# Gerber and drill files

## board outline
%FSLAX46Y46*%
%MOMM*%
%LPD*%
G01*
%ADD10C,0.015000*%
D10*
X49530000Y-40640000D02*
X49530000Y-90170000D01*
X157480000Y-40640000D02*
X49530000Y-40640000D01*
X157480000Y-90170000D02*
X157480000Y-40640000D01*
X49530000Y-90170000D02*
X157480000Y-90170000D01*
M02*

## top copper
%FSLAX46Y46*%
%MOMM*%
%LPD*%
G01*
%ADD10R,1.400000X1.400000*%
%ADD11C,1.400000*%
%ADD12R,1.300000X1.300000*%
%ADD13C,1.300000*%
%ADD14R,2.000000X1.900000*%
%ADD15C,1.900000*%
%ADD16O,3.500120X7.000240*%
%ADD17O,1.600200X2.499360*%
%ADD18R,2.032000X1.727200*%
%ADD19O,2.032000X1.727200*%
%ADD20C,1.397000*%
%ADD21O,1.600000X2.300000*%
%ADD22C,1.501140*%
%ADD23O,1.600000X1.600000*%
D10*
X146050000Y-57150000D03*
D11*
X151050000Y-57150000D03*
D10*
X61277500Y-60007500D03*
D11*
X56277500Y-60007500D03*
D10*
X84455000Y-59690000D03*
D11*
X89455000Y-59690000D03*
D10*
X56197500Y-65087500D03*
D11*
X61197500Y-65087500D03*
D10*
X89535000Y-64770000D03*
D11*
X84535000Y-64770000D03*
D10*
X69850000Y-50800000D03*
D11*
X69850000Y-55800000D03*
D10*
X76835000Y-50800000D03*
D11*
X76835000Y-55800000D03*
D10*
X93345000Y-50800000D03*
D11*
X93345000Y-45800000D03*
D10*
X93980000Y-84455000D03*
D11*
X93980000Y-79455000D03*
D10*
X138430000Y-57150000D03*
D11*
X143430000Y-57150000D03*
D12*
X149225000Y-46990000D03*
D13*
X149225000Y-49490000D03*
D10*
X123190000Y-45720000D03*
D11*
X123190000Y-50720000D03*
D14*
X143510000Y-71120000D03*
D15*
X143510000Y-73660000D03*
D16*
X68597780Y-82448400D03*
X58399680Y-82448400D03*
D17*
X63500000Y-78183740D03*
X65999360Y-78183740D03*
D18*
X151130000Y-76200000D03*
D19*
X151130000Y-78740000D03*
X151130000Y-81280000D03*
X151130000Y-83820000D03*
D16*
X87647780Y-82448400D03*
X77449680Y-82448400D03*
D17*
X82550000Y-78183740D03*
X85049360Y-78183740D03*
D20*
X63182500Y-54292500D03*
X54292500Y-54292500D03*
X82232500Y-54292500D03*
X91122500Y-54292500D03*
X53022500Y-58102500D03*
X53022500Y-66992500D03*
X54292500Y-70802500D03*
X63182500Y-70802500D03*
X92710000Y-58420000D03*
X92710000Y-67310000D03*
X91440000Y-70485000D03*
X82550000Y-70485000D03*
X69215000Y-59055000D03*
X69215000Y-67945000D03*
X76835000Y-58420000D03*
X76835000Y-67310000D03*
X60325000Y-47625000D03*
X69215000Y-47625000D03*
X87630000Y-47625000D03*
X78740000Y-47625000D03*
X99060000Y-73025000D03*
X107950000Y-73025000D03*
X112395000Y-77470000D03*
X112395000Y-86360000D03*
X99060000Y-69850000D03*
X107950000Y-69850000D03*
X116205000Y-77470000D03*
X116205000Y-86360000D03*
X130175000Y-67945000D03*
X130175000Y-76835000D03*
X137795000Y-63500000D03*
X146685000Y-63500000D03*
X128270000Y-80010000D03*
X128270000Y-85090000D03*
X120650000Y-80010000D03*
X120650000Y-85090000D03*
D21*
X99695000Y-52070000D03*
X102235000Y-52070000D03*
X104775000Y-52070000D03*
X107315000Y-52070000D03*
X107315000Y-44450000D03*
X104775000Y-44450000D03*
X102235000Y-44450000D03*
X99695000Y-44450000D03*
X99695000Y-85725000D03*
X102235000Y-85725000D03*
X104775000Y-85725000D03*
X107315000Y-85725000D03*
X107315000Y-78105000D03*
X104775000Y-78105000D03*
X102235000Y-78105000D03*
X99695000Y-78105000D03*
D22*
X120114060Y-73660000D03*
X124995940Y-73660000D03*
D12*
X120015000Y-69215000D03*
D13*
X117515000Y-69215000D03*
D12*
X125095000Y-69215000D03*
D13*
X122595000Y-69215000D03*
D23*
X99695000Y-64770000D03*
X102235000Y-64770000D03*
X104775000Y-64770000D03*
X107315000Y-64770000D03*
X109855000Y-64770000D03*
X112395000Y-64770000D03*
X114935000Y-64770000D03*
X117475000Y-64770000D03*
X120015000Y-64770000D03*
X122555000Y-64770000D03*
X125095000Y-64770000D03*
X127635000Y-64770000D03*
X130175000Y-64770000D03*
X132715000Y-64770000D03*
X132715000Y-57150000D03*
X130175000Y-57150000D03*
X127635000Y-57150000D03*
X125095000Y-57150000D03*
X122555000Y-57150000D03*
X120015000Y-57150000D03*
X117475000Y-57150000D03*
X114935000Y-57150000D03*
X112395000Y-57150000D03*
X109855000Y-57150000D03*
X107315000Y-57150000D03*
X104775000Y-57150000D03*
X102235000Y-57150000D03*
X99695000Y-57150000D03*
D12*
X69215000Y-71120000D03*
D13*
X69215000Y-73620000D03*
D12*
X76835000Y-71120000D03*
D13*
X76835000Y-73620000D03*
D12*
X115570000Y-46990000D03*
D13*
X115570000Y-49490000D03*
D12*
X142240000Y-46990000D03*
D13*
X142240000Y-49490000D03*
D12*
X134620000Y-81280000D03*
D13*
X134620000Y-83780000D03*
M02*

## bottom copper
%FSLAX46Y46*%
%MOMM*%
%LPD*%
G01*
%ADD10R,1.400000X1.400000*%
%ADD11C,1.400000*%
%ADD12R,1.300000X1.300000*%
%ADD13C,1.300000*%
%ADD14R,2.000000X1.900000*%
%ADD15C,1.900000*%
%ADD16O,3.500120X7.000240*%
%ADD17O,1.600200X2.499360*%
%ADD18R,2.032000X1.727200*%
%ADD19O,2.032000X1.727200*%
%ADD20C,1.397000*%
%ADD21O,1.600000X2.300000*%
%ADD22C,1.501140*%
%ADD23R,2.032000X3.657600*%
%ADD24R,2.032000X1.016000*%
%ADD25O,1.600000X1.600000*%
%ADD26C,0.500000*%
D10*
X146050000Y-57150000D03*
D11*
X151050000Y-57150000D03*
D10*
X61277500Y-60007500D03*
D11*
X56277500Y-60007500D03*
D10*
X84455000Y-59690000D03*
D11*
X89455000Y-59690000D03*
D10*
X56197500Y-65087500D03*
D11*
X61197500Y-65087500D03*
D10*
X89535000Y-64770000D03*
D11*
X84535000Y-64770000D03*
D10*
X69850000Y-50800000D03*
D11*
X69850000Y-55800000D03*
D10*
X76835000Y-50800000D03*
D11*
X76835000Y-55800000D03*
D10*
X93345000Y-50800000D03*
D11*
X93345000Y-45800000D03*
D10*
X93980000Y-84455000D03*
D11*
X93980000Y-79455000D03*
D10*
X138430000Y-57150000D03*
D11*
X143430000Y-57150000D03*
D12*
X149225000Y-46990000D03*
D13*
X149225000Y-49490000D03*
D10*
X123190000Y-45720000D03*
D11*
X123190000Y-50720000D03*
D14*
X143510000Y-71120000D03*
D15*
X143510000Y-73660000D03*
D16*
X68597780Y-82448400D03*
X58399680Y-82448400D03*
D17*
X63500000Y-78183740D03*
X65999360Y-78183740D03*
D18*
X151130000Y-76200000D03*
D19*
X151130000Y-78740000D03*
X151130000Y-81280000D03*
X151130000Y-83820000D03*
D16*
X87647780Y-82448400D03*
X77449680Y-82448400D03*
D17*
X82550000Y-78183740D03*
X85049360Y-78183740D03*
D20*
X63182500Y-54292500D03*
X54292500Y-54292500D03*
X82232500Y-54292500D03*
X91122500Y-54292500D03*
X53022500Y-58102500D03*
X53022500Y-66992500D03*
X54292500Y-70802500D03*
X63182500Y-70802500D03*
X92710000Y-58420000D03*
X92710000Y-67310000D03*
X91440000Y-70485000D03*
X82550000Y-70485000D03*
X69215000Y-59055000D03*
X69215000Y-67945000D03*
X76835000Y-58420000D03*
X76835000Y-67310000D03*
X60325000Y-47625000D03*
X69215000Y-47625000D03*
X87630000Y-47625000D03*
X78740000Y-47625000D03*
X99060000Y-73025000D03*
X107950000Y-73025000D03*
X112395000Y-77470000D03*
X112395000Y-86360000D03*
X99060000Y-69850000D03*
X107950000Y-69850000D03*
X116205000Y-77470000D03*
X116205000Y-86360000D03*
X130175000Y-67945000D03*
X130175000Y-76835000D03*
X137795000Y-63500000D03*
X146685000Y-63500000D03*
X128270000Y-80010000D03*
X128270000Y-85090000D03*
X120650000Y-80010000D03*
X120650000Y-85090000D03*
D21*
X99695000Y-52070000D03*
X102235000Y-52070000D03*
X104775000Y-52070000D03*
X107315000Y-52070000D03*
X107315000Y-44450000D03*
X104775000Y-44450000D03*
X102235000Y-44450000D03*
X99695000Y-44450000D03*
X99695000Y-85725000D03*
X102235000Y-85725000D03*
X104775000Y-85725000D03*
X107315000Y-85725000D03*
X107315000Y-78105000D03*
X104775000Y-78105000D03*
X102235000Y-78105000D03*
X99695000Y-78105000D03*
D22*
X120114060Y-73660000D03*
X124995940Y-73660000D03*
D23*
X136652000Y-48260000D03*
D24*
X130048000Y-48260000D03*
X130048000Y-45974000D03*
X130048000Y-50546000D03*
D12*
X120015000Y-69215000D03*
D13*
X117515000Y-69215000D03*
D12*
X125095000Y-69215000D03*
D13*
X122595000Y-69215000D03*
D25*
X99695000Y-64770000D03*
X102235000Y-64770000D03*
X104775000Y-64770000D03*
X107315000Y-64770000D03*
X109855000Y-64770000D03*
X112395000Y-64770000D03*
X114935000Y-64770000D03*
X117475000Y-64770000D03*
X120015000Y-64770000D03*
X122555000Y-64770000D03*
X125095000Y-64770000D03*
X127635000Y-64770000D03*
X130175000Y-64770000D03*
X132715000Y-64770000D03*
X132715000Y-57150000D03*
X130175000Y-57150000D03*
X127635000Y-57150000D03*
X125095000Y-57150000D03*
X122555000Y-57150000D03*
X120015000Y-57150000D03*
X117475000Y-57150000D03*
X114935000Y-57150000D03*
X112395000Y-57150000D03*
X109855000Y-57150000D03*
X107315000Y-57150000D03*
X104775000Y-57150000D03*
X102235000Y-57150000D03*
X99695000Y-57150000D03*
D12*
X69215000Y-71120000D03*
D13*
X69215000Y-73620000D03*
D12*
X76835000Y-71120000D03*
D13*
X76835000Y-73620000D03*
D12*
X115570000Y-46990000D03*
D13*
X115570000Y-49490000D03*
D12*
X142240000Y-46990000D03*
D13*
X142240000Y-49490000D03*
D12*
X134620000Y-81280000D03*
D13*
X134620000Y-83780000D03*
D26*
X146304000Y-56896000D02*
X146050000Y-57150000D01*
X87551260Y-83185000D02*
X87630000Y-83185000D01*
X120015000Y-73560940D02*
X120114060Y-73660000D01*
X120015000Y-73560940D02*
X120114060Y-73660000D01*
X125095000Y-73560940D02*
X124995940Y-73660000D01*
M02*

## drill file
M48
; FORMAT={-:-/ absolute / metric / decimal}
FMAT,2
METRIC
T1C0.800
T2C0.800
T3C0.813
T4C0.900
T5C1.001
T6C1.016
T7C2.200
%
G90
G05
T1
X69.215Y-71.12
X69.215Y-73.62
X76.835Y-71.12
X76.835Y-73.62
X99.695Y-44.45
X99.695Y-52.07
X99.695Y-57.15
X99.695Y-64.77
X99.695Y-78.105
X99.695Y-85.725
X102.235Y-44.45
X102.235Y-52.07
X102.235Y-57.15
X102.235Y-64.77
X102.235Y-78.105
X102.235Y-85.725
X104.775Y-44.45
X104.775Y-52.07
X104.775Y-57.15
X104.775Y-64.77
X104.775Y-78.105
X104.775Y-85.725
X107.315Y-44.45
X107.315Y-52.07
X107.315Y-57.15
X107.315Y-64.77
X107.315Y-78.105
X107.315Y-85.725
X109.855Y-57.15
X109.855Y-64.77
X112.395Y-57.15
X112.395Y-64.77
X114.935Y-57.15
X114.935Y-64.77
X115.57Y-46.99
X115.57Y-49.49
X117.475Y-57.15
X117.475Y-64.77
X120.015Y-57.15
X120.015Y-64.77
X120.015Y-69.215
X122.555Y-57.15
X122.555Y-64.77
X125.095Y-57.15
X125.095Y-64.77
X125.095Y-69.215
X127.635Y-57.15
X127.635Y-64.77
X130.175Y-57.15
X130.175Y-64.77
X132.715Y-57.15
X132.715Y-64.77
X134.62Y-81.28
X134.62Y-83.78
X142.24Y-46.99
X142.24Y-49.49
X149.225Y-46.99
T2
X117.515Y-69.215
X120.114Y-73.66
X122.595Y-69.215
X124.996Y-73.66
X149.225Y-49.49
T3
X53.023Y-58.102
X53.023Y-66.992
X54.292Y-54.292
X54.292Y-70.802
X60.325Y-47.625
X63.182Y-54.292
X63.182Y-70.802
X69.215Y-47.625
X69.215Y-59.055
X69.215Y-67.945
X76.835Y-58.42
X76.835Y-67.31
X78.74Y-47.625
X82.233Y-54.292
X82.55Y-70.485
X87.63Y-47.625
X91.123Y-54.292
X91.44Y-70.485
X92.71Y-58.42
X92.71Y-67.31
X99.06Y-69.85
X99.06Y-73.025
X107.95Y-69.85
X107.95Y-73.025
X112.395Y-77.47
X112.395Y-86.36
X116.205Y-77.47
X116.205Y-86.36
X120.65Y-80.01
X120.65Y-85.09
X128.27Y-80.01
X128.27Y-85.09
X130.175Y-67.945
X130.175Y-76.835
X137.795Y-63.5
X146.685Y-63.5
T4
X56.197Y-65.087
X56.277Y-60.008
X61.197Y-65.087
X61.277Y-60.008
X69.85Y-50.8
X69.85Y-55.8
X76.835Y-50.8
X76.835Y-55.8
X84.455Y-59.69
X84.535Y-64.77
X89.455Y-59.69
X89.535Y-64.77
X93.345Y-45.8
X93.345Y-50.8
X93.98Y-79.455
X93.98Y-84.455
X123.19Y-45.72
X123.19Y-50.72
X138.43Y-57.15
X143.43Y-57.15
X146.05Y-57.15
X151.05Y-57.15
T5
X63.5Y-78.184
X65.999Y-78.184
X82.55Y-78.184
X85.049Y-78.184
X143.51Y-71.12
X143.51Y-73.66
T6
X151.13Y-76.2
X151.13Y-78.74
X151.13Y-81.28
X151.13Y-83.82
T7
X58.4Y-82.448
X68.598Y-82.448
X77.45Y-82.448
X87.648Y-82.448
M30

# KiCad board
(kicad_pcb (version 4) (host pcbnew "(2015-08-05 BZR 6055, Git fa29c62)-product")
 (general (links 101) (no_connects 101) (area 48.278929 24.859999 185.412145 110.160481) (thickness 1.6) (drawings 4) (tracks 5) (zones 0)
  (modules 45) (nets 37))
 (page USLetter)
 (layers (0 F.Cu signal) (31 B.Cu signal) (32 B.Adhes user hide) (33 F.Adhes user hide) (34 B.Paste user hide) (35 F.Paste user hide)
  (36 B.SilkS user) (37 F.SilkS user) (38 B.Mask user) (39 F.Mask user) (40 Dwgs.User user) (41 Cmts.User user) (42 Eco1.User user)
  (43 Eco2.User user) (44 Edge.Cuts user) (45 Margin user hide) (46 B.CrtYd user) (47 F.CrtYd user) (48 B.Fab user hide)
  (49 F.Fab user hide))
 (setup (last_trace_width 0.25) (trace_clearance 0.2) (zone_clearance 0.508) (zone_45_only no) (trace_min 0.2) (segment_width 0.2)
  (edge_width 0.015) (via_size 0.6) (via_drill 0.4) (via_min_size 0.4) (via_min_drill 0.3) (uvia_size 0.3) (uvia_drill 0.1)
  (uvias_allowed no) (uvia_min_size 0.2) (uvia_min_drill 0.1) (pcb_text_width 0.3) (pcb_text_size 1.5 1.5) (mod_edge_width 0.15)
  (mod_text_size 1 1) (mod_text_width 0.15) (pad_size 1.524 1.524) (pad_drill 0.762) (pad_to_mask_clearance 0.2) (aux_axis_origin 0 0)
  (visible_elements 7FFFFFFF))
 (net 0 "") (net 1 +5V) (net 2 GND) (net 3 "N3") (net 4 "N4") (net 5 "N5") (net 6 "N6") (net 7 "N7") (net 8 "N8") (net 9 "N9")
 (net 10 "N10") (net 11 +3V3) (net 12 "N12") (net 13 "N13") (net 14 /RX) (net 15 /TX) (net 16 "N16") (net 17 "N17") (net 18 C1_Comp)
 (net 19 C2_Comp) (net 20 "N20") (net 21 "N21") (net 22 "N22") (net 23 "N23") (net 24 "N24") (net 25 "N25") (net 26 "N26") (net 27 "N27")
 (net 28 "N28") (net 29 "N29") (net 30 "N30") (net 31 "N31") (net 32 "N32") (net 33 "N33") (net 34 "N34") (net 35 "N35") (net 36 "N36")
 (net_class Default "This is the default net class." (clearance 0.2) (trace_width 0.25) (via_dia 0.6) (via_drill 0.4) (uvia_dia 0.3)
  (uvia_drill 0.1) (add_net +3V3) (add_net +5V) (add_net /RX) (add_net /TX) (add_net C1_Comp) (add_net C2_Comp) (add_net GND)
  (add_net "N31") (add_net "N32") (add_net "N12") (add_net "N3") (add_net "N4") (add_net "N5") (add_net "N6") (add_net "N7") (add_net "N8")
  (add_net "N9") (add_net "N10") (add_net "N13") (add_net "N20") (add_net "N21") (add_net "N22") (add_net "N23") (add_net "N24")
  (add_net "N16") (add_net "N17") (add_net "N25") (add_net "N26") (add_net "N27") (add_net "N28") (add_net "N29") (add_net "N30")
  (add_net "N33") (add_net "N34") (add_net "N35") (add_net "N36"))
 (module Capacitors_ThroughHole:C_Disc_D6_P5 (layer F.Cu) (at 146.05 57.15)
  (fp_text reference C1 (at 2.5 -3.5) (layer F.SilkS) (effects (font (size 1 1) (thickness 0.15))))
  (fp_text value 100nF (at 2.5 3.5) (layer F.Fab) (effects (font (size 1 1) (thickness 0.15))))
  (pad 1 thru_hole rect (at 0 0) (size 1.4 1.4) (drill 0.9) (layers *.Cu *.Mask F.SilkS) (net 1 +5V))
  (pad 2 thru_hole circle (at 5 0) (size 1.4 1.4) (drill 0.9) (layers *.Cu *.Mask F.SilkS) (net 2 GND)))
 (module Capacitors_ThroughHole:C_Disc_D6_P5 (layer F.Cu) (at 61.2775 60.0075 180)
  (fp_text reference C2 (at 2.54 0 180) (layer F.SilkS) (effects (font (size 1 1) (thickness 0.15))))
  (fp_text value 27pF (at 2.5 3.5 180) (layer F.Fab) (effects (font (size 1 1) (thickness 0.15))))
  (pad 1 thru_hole rect (at 0 0 180) (size 1.4 1.4) (drill 0.9) (layers *.Cu *.Mask F.SilkS) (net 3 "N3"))
  (pad 2 thru_hole circle (at 5 0 180) (size 1.4 1.4) (drill 0.9) (layers *.Cu *.Mask F.SilkS) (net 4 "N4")))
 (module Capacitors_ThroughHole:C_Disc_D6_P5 (layer F.Cu) (at 84.455 59.69)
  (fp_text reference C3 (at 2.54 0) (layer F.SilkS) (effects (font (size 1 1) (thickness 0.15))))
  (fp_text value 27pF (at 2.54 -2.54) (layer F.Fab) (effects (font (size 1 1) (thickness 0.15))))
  (pad 1 thru_hole rect (at 0 0) (size 1.4 1.4) (drill 0.9) (layers *.Cu *.Mask F.SilkS) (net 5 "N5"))
  (pad 2 thru_hole circle (at 5 0) (size 1.4 1.4) (drill 0.9) (layers *.Cu *.Mask F.SilkS) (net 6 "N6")))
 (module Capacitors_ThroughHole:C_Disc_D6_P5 (layer F.Cu) (at 56.1975 65.0875)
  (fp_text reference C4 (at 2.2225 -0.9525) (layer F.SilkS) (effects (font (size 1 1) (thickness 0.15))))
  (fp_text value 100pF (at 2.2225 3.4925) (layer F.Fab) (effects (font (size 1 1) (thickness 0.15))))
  (pad 1 thru_hole rect (at 0 0) (size 1.4 1.4) (drill 0.9) (layers *.Cu *.Mask F.SilkS) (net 4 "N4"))
  (pad 2 thru_hole circle (at 5 0) (size 1.4 1.4) (drill 0.9) (layers *.Cu *.Mask F.SilkS) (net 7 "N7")))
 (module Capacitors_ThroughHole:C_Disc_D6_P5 (layer F.Cu) (at 89.535 64.77 180)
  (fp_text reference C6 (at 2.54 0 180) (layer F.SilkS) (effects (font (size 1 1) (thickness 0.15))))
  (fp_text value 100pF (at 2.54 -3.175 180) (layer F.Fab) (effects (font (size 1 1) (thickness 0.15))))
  (pad 1 thru_hole rect (at 0 0 180) (size 1.4 1.4) (drill 0.9) (layers *.Cu *.Mask F.SilkS) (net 6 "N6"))
  (pad 2 thru_hole circle (at 5 0 180) (size 1.4 1.4) (drill 0.9) (layers *.Cu *.Mask F.SilkS) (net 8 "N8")))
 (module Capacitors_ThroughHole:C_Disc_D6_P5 (layer F.Cu) (at 69.85 50.8 270)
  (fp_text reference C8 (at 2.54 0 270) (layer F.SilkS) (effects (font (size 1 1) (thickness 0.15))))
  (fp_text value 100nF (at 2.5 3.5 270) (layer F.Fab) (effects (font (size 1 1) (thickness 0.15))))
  (pad 1 thru_hole rect (at 0 0 270) (size 1.4 1.4) (drill 0.9) (layers *.Cu *.Mask F.SilkS) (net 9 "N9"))
  (pad 2 thru_hole circle (at 5 0 270) (size 1.4 1.4) (drill 0.9) (layers *.Cu *.Mask F.SilkS) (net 2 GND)))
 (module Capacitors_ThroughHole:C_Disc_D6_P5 (layer F.Cu) (at 76.835 50.8 270)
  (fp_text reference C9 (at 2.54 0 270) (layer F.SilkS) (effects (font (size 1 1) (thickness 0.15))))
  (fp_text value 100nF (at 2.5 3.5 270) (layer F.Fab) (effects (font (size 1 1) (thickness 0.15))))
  (pad 1 thru_hole rect (at 0 0 270) (size 1.4 1.4) (drill 0.9) (layers *.Cu *.Mask F.SilkS) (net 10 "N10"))
  (pad 2 thru_hole circle (at 5 0 270) (size 1.4 1.4) (drill 0.9) (layers *.Cu *.Mask F.SilkS) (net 2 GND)))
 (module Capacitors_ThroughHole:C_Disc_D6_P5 (layer F.Cu) (at 93.345 50.8 90)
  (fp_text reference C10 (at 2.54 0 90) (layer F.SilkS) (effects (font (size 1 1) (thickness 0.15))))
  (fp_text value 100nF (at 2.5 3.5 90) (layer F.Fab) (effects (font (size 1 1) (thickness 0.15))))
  (pad 1 thru_hole rect (at 0 0 90) (size 1.4 1.4) (drill 0.9) (layers *.Cu *.Mask F.SilkS) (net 2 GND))
  (pad 2 thru_hole circle (at 5 0 90) (size 1.4 1.4) (drill 0.9) (layers *.Cu *.Mask F.SilkS) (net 1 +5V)))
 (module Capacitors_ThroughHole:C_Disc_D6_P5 (layer F.Cu) (at 93.98 84.455 90)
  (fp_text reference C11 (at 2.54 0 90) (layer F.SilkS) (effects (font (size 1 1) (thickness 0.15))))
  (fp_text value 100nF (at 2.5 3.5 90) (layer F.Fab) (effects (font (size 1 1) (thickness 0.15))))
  (pad 1 thru_hole rect (at 0 0 90) (size 1.4 1.4) (drill 0.9) (layers *.Cu *.Mask F.SilkS) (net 2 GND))
  (pad 2 thru_hole circle (at 5 0 90) (size 1.4 1.4) (drill 0.9) (layers *.Cu *.Mask F.SilkS) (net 1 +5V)))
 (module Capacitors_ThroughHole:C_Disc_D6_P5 (layer F.Cu) (at 138.43 57.15)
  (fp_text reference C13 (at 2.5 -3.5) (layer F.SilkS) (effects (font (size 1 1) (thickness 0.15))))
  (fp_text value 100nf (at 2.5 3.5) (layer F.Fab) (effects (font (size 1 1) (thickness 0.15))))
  (pad 1 thru_hole rect (at 0 0) (size 1.4 1.4) (drill 0.9) (layers *.Cu *.Mask F.SilkS) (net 1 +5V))
  (pad 2 thru_hole circle (at 5 0) (size 1.4 1.4) (drill 0.9) (layers *.Cu *.Mask F.SilkS) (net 2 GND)))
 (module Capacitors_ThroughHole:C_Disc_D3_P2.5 (layer F.Cu) (at 149.225 46.99 270)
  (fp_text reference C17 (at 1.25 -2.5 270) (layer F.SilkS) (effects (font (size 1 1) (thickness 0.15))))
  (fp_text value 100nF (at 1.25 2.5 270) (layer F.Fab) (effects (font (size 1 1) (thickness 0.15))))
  (pad 1 thru_hole rect (at 0 0 270) (size 1.3 1.3) (drill 0.8) (layers *.Cu *.Mask F.SilkS) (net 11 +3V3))
  (pad 2 thru_hole circle (at 2.5 0 270) (size 1.3 1.3) (drill 0.8001) (layers *.Cu *.Mask F.SilkS) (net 2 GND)))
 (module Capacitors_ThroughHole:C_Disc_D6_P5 (layer F.Cu) (at 123.19 45.72 270)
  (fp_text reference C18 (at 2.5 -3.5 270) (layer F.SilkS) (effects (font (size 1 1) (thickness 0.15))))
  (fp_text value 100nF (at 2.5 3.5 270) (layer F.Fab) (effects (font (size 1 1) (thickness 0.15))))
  (pad 1 thru_hole rect (at 0 0 270) (size 1.4 1.4) (drill 0.9) (layers *.Cu *.Mask F.SilkS) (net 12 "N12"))
  (pad 2 thru_hole circle (at 5 0 270) (size 1.4 1.4) (drill 0.9) (layers *.Cu *.Mask F.SilkS) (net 2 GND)))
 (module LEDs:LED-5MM (layer F.Cu) (at 143.51 71.12 270)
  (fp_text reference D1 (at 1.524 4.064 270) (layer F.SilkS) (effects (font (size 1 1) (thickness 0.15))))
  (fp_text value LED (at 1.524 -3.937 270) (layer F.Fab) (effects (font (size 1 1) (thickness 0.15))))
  (pad 1 thru_hole rect (at 0 0) (size 2 1.9) (drill 1.00076) (layers *.Cu *.Mask F.SilkS) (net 2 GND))
  (pad 2 thru_hole circle (at 2.54 0 270) (size 1.9 1.9) (drill 1.00076) (layers *.Cu *.Mask F.SilkS) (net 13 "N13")))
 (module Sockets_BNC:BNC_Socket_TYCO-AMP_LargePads (layer F.Cu) (at 63.5 83.185 180)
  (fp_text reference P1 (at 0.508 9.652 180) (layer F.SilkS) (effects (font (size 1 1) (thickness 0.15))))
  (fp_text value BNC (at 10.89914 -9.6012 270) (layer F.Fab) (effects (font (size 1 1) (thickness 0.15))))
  (pad 2 thru_hole oval (at -5.09778 0.7366 180) (size 3.50012 7.00024) (drill 2.19964) (layers *.Cu *.Mask F.SilkS) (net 2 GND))
  (pad 2 thru_hole oval (at 5.10032 0.7366 180) (size 3.50012 7.00024) (drill 2.19964) (layers *.Cu *.Mask F.SilkS) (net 2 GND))
  (pad 1 thru_hole oval (at 0 5.00126 180) (size 1.6002 2.49936) (drill 1.00076) (layers *.Cu *.Mask F.SilkS) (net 3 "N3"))
  (pad 2 thru_hole oval (at -2.49936 5.00126 180) (size 1.6002 2.49936) (drill 1.00076) (layers *.Cu *.Mask F.SilkS) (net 2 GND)))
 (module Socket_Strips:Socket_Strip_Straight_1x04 (layer F.Cu) (at 151.13 76.2 270)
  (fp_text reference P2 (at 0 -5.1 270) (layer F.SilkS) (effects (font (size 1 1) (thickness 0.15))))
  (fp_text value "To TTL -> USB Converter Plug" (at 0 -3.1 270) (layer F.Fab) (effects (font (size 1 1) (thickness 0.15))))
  (pad 1 thru_hole rect (at 0 0 270) (size 1.7272 2.032) (drill 1.016) (layers *.Cu *.Mask F.SilkS) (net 2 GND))
  (pad 2 thru_hole oval (at 2.54 0 270) (size 1.7272 2.032) (drill 1.016) (layers *.Cu *.Mask F.SilkS) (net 1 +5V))
  (pad 3 thru_hole oval (at 5.08 0 270) (size 1.7272 2.032) (drill 1.016) (layers *.Cu *.Mask F.SilkS) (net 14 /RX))
  (pad 4 thru_hole oval (at 7.62 0 270) (size 1.7272 2.032) (drill 1.016) (layers *.Cu *.Mask F.SilkS) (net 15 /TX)))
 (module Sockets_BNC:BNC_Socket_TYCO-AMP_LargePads (layer F.Cu) (at 82.55 83.185 180)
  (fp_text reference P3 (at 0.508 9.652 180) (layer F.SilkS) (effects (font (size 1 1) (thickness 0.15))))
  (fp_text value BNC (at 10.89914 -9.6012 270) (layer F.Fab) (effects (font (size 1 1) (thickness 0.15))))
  (pad 2 thru_hole oval (at -5.09778 0.7366 180) (size 3.50012 7.00024) (drill 2.19964) (layers *.Cu *.Mask F.SilkS) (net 2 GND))
  (pad 2 thru_hole oval (at 5.10032 0.7366 180) (size 3.50012 7.00024) (drill 2.19964) (layers *.Cu *.Mask F.SilkS) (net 2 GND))
  (pad 1 thru_hole oval (at 0 5.00126 180) (size 1.6002 2.49936) (drill 1.00076) (layers *.Cu *.Mask F.SilkS) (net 5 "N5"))
  (pad 2 thru_hole oval (at -2.49936 5.00126 180) (size 1.6002 2.49936) (drill 1.00076) (layers *.Cu *.Mask F.SilkS) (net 2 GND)))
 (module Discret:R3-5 (layer F.Cu) (at 58.7375 54.2925 180)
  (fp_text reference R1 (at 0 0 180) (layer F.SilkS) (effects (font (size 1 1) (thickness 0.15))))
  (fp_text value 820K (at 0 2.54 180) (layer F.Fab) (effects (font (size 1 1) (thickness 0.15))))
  (pad 1 thru_hole circle (at -4.445 0 180) (size 1.397 1.397) (drill 0.8128) (layers *.Cu *.Mask F.SilkS) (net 3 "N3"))
  (pad 2 thru_hole circle (at 4.445 0 180) (size 1.397 1.397) (drill 0.8128) (layers *.Cu *.Mask F.SilkS) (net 4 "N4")))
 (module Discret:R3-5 (layer F.Cu) (at 86.6775 54.2925)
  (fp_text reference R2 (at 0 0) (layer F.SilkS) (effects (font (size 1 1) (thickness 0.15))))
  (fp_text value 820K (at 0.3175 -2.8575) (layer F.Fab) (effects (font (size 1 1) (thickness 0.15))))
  (pad 1 thru_hole circle (at -4.445 0) (size 1.397 1.397) (drill 0.8128) (layers *.Cu *.Mask F.SilkS) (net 5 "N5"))
  (pad 2 thru_hole circle (at 4.445 0) (size 1.397 1.397) (drill 0.8128) (layers *.Cu *.Mask F.SilkS) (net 6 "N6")))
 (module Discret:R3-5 (layer F.Cu) (at 53.0225 62.5475 270)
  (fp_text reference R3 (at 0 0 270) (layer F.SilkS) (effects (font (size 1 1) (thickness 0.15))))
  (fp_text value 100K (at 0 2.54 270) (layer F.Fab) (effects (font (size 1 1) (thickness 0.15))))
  (pad 1 thru_hole circle (at -4.445 0 270) (size 1.397 1.397) (drill 0.8128) (layers *.Cu *.Mask F.SilkS) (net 4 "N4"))
  (pad 2 thru_hole circle (at 4.445 0 270) (size 1.397 1.397) (drill 0.8128) (layers *.Cu *.Mask F.SilkS) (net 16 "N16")))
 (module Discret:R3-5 (layer F.Cu) (at 58.7375 70.8025)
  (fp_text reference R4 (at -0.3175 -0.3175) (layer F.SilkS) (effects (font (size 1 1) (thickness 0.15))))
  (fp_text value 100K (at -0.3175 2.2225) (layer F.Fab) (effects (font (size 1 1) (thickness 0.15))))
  (pad 1 thru_hole circle (at -4.445 0) (size 1.397 1.397) (drill 0.8128) (layers *.Cu *.Mask F.SilkS) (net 16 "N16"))
  (pad 2 thru_hole circle (at 4.445 0) (size 1.397 1.397) (drill 0.8128) (layers *.Cu *.Mask F.SilkS) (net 7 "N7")))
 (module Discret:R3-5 (layer F.Cu) (at 92.71 62.865 270)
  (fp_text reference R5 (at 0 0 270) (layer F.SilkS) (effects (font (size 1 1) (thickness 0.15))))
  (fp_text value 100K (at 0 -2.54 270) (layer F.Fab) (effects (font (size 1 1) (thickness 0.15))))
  (pad 1 thru_hole circle (at -4.445 0 270) (size 1.397 1.397) (drill 0.8128) (layers *.Cu *.Mask F.SilkS) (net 6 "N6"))
  (pad 2 thru_hole circle (at 4.445 0 270) (size 1.397 1.397) (drill 0.8128) (layers *.Cu *.Mask F.SilkS) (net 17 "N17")))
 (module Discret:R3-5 (layer F.Cu) (at 86.995 70.485 180)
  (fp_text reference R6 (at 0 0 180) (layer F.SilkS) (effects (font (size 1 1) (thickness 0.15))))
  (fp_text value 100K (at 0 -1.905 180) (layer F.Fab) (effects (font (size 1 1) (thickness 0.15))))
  (pad 1 thru_hole circle (at -4.445 0 180) (size 1.397 1.397) (drill 0.8128) (layers *.Cu *.Mask F.SilkS) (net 17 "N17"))
  (pad 2 thru_hole circle (at 4.445 0 180) (size 1.397 1.397) (drill 0.8128) (layers *.Cu *.Mask F.SilkS) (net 8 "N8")))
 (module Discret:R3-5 (layer F.Cu) (at 69.215 63.5 270)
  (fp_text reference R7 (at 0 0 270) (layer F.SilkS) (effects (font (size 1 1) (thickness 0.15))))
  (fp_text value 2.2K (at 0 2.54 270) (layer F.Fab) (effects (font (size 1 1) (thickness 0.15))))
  (pad 1 thru_hole circle (at -4.445 0 270) (size 1.397 1.397) (drill 0.8128) (layers *.Cu *.Mask F.SilkS) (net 9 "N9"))
  (pad 2 thru_hole circle (at 4.445 0 270) (size 1.397 1.397) (drill 0.8128) (layers *.Cu *.Mask F.SilkS) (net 7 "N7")))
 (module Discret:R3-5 (layer F.Cu) (at 76.835 62.865 270)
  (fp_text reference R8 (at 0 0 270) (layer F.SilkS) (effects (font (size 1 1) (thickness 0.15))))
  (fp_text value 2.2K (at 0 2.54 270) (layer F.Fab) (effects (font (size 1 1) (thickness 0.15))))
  (pad 1 thru_hole circle (at -4.445 0 270) (size 1.397 1.397) (drill 0.8128) (layers *.Cu *.Mask F.SilkS) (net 10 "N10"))
  (pad 2 thru_hole circle (at 4.445 0 270) (size 1.397 1.397) (drill 0.8128) (layers *.Cu *.Mask F.SilkS) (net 8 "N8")))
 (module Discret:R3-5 (layer F.Cu) (at 64.77 47.625)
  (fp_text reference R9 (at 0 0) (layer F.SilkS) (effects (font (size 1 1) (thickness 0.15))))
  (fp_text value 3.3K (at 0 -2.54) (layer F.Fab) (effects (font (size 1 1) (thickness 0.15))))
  (pad 1 thru_hole circle (at -4.445 0) (size 1.397 1.397) (drill 0.8128) (layers *.Cu *.Mask F.SilkS) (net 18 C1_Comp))
  (pad 2 thru_hole circle (at 4.445 0) (size 1.397 1.397) (drill 0.8128) (layers *.Cu *.Mask F.SilkS) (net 9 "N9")))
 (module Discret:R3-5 (layer F.Cu) (at 83.185 47.625 180)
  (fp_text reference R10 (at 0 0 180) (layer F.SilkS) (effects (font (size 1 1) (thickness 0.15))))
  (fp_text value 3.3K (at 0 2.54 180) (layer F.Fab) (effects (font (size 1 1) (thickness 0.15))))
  (pad 1 thru_hole circle (at -4.445 0 180) (size 1.397 1.397) (drill 0.8128) (layers *.Cu *.Mask F.SilkS) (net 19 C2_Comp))
  (pad 2 thru_hole circle (at 4.445 0 180) (size 1.397 1.397) (drill 0.8128) (layers *.Cu *.Mask F.SilkS) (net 10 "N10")))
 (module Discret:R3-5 (layer F.Cu) (at 103.505 73.025)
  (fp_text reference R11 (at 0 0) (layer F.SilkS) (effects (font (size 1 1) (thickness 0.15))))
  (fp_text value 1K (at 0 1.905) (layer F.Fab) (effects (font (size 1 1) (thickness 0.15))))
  (pad 1 thru_hole circle (at -4.445 0) (size 1.397 1.397) (drill 0.8128) (layers *.Cu *.Mask F.SilkS) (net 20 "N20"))
  (pad 2 thru_hole circle (at 4.445 0) (size 1.397 1.397) (drill 0.8128) (layers *.Cu *.Mask F.SilkS) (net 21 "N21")))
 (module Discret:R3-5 (layer F.Cu) (at 112.395 81.915 270)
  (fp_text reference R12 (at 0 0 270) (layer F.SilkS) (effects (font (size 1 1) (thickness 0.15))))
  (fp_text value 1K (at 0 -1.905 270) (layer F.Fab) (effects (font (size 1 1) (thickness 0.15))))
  (pad 1 thru_hole circle (at -4.445 0 270) (size 1.397 1.397) (drill 0.8128) (layers *.Cu *.Mask F.SilkS) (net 21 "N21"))
  (pad 2 thru_hole circle (at 4.445 0 270) (size 1.397 1.397) (drill 0.8128) (layers *.Cu *.Mask F.SilkS) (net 2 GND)))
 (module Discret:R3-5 (layer F.Cu) (at 103.505 69.85)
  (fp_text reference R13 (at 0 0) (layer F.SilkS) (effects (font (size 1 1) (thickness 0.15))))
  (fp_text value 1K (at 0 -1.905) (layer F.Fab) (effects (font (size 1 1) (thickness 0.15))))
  (pad 1 thru_hole circle (at -4.445 0) (size 1.397 1.397) (drill 0.8128) (layers *.Cu *.Mask F.SilkS) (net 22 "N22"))
  (pad 2 thru_hole circle (at 4.445 0) (size 1.397 1.397) (drill 0.8128) (layers *.Cu *.Mask F.SilkS) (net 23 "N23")))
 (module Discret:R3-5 (layer F.Cu) (at 116.205 81.915 270)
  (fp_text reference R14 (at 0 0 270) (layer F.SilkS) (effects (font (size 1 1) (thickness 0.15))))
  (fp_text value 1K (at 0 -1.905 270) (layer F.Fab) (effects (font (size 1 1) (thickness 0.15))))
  (pad 1 thru_hole circle (at -4.445 0 270) (size 1.397 1.397) (drill 0.8128) (layers *.Cu *.Mask F.SilkS) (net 23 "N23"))
  (pad 2 thru_hole circle (at 4.445 0 270) (size 1.397 1.397) (drill 0.8128) (layers *.Cu *.Mask F.SilkS) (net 2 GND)))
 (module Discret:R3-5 (layer F.Cu) (at 130.175 72.39 270)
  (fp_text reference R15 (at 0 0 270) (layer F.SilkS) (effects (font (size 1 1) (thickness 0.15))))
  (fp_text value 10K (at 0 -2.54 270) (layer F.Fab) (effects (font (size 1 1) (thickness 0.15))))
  (pad 1 thru_hole circle (at -4.445 0 270) (size 1.397 1.397) (drill 0.8128) (layers *.Cu *.Mask F.SilkS) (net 1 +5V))
  (pad 2 thru_hole circle (at 4.445 0 270) (size 1.397 1.397) (drill 0.8128) (layers *.Cu *.Mask F.SilkS) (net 12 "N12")))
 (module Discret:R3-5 (layer F.Cu) (at 142.24 63.5)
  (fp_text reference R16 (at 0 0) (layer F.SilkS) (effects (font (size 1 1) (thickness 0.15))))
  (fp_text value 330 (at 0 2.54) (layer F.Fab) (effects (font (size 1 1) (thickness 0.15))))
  (pad 1 thru_hole circle (at -4.445 0) (size 1.397 1.397) (drill 0.8128) (layers *.Cu *.Mask F.SilkS) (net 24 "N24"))
  (pad 2 thru_hole circle (at 4.445 0) (size 1.397 1.397) (drill 0.8128) (layers *.Cu *.Mask F.SilkS) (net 13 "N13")))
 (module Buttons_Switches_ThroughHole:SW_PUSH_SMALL (layer F.Cu) (at 124.46 82.55)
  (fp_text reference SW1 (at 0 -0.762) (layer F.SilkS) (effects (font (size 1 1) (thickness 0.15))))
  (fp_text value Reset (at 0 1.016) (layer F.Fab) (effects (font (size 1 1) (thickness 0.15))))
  (pad 1 thru_hole circle (at 3.81 -2.54) (size 1.397 1.397) (drill 0.8128) (layers *.Cu *.Mask F.SilkS) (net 12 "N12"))
  (pad 2 thru_hole circle (at 3.81 2.54) (size 1.397 1.397) (drill 0.8128) (layers *.Cu *.Mask F.SilkS) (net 2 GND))
  (pad 1 thru_hole circle (at -3.81 -2.54) (size 1.397 1.397) (drill 0.8128) (layers *.Cu *.Mask F.SilkS) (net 12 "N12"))
  (pad 2 thru_hole circle (at -3.81 2.54) (size 1.397 1.397) (drill 0.8128) (layers *.Cu *.Mask F.SilkS) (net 2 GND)))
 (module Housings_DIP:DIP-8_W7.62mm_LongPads (layer F.Cu) (at 99.695 52.07 90)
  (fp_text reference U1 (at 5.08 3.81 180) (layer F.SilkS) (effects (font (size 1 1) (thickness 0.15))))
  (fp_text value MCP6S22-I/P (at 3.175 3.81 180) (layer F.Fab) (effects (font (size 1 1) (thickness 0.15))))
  (pad 1 thru_hole oval (at 0 0 90) (size 2.3 1.6) (drill 0.8) (layers *.Cu *.Mask F.SilkS) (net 20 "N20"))
  (pad 2 thru_hole oval (at 0 2.54 90) (size 2.3 1.6) (drill 0.8) (layers *.Cu *.Mask F.SilkS) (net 4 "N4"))
  (pad 3 thru_hole oval (at 0 5.08 90) (size 2.3 1.6) (drill 0.8) (layers *.Cu *.Mask F.SilkS) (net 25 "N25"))
  (pad 4 thru_hole oval (at 0 7.62 90) (size 2.3 1.6) (drill 0.8) (layers *.Cu *.Mask F.SilkS) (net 2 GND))
  (pad 5 thru_hole oval (at 7.62 7.62 90) (size 2.3 1.6) (drill 0.8) (layers *.Cu *.Mask F.SilkS) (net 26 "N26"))
  (pad 6 thru_hole oval (at 7.62 5.08 90) (size 2.3 1.6) (drill 0.8) (layers *.Cu *.Mask F.SilkS) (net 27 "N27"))
  (pad 7 thru_hole oval (at 7.62 2.54 90) (size 2.3 1.6) (drill 0.8) (layers *.Cu *.Mask F.SilkS) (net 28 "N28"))
  (pad 8 thru_hole oval (at 7.62 0 90) (size 2.3 1.6) (drill 0.8) (layers *.Cu *.Mask F.SilkS) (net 1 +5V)))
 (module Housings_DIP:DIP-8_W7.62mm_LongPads (layer F.Cu) (at 99.695 85.725 90)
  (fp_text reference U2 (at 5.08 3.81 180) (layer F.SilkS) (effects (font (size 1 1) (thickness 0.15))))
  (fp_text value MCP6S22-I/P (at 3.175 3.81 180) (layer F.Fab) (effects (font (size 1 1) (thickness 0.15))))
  (pad 1 thru_hole oval (at 0 0 90) (size 2.3 1.6) (drill 0.8) (layers *.Cu *.Mask F.SilkS) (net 22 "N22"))
  (pad 2 thru_hole oval (at 0 2.54 90) (size 2.3 1.6) (drill 0.8) (layers *.Cu *.Mask F.SilkS) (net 6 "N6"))
  (pad 3 thru_hole oval (at 0 5.08 90) (size 2.3 1.6) (drill 0.8) (layers *.Cu *.Mask F.SilkS) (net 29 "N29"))
  (pad 4 thru_hole oval (at 0 7.62 90) (size 2.3 1.6) (drill 0.8) (layers *.Cu *.Mask F.SilkS) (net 2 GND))
  (pad 5 thru_hole oval (at 7.62 7.62 90) (size 2.3 1.6) (drill 0.8) (layers *.Cu *.Mask F.SilkS) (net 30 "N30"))
  (pad 6 thru_hole oval (at 7.62 5.08 90) (size 2.3 1.6) (drill 0.8) (layers *.Cu *.Mask F.SilkS) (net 27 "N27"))
  (pad 7 thru_hole oval (at 7.62 2.54 90) (size 2.3 1.6) (drill 0.8) (layers *.Cu *.Mask F.SilkS) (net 28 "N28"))
  (pad 8 thru_hole oval (at 7.62 0 90) (size 2.3 1.6) (drill 0.8) (layers *.Cu *.Mask F.SilkS) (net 1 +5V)))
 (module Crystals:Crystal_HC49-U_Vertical (layer F.Cu) (at 122.555 73.66)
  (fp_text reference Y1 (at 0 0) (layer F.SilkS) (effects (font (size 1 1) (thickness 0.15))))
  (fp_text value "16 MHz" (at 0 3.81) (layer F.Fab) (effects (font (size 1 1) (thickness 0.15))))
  (pad 1 thru_hole circle (at -2.44094 0) (size 1.50114 1.50114) (drill 0.8001) (layers *.Cu *.Mask F.SilkS) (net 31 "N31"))
  (pad 2 thru_hole circle (at 2.44094 0) (size 1.50114 1.50114) (drill 0.8001) (layers *.Cu *.Mask F.SilkS) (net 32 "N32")))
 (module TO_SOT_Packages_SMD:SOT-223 (layer B.Cu) (at 133.35 48.26 90)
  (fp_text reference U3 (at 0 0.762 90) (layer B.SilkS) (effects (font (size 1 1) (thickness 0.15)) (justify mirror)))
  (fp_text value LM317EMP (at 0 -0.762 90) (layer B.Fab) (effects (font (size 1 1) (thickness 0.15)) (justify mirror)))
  (pad 4 smd rect (at 0 3.302 90) (size 3.6576 2.032) (layers B.Cu B.Paste B.Mask))
  (pad 2 smd rect (at 0 -3.302 90) (size 1.016 2.032) (layers B.Cu B.Paste B.Mask) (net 11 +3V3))
  (pad 3 smd rect (at 2.286 -3.302 90) (size 1.016 2.032) (layers B.Cu B.Paste B.Mask) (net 1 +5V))
  (pad 1 smd rect (at -2.286 -3.302 90) (size 1.016 2.032) (layers B.Cu B.Paste B.Mask) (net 2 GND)))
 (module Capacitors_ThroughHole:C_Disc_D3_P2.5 (layer F.Cu) (at 120.015 69.215 180)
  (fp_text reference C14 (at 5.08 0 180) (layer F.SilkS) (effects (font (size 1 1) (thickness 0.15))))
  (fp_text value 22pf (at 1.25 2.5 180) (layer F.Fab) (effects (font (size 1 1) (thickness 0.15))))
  (pad 1 thru_hole rect (at 0 0 180) (size 1.3 1.3) (drill 0.8) (layers *.Cu *.Mask F.SilkS) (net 31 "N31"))
  (pad 2 thru_hole circle (at 2.5 0 180) (size 1.3 1.3) (drill 0.8001) (layers *.Cu *.Mask F.SilkS) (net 2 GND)))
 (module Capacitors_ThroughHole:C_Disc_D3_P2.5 (layer F.Cu) (at 125.095 69.215 180)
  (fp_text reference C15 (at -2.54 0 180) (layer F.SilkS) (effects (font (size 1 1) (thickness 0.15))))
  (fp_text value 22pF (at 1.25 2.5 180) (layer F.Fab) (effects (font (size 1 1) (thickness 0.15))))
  (pad 1 thru_hole rect (at 0 0 180) (size 1.3 1.3) (drill 0.8) (layers *.Cu *.Mask F.SilkS) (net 32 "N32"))
  (pad 2 thru_hole circle (at 2.5 0 180) (size 1.3 1.3) (drill 0.8001) (layers *.Cu *.Mask F.SilkS) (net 2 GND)))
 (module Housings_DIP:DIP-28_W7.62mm (layer F.Cu) (at 99.695 64.77 90)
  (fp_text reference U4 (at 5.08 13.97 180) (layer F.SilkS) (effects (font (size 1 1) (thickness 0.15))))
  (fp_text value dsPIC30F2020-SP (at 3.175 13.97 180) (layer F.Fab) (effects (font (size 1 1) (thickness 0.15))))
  (pad 1 thru_hole oval (at 0 0 90) (size 1.6 1.6) (drill 0.8) (layers *.Cu *.Mask F.SilkS) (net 12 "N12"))
  (pad 2 thru_hole oval (at 0 2.54 90) (size 1.6 1.6) (drill 0.8) (layers *.Cu *.Mask F.SilkS) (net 20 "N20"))
  (pad 3 thru_hole oval (at 0 5.08 90) (size 1.6 1.6) (drill 0.8) (layers *.Cu *.Mask F.SilkS) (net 22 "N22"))
  (pad 4 thru_hole oval (at 0 7.62 90) (size 1.6 1.6) (drill 0.8) (layers *.Cu *.Mask F.SilkS) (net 11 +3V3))
  (pad 5 thru_hole oval (at 0 10.16 90) (size 1.6 1.6) (drill 0.8) (layers *.Cu *.Mask F.SilkS) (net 11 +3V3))
  (pad 6 thru_hole oval (at 0 12.7 90) (size 1.6 1.6) (drill 0.8) (layers *.Cu *.Mask F.SilkS) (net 21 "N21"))
  (pad 7 thru_hole oval (at 0 15.24 90) (size 1.6 1.6) (drill 0.8) (layers *.Cu *.Mask F.SilkS) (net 23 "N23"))
  (pad 8 thru_hole oval (at 0 17.78 90) (size 1.6 1.6) (drill 0.8) (layers *.Cu *.Mask F.SilkS) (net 2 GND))
  (pad 9 thru_hole oval (at 0 20.32 90) (size 1.6 1.6) (drill 0.8) (layers *.Cu *.Mask F.SilkS) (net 31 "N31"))
  (pad 10 thru_hole oval (at 0 22.86 90) (size 1.6 1.6) (drill 0.8) (layers *.Cu *.Mask F.SilkS) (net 32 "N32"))
  (pad 11 thru_hole oval (at 0 25.4 90) (size 1.6 1.6) (drill 0.8) (layers *.Cu *.Mask F.SilkS) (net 15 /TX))
  (pad 12 thru_hole oval (at 0 27.94 90) (size 1.6 1.6) (drill 0.8) (layers *.Cu *.Mask F.SilkS) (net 14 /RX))
  (pad 13 thru_hole oval (at 0 30.48 90) (size 1.6 1.6) (drill 0.8) (layers *.Cu *.Mask F.SilkS) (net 1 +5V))
  (pad 14 thru_hole oval (at 0 33.02 90) (size 1.6 1.6) (drill 0.8) (layers *.Cu *.Mask F.SilkS) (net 19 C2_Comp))
  (pad 15 thru_hole oval (at 7.62 33.02 90) (size 1.6 1.6) (drill 0.8) (layers *.Cu *.Mask F.SilkS) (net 18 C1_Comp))
  (pad 16 thru_hole oval (at 7.62 30.48 90) (size 1.6 1.6) (drill 0.8) (layers *.Cu *.Mask F.SilkS) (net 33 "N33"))
  (pad 17 thru_hole oval (at 7.62 27.94 90) (size 1.6 1.6) (drill 0.8) (layers *.Cu *.Mask F.SilkS) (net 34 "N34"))
  (pad 18 thru_hole oval (at 7.62 25.4 90) (size 1.6 1.6) (drill 0.8) (layers *.Cu *.Mask F.SilkS) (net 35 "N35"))
  (pad 19 thru_hole oval (at 7.62 22.86 90) (size 1.6 1.6) (drill 0.8) (layers *.Cu *.Mask F.SilkS) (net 2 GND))
  (pad 20 thru_hole oval (at 7.62 20.32 90) (size 1.6 1.6) (drill 0.8) (layers *.Cu *.Mask F.SilkS) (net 1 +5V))
  (pad 21 thru_hole oval (at 7.62 17.78 90) (size 1.6 1.6) (drill 0.8) (layers *.Cu *.Mask F.SilkS) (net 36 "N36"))
  (pad 22 thru_hole oval (at 7.62 15.24 90) (size 1.6 1.6) (drill 0.8) (layers *.Cu *.Mask F.SilkS) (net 24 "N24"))
  (pad 23 thru_hole oval (at 7.62 12.7 90) (size 1.6 1.6) (drill 0.8) (layers *.Cu *.Mask F.SilkS) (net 30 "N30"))
  (pad 24 thru_hole oval (at 7.62 10.16 90) (size 1.6 1.6) (drill 0.8) (layers *.Cu *.Mask F.SilkS) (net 26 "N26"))
  (pad 25 thru_hole oval (at 7.62 7.62 90) (size 1.6 1.6) (drill 0.8) (layers *.Cu *.Mask F.SilkS) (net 27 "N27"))
  (pad 26 thru_hole oval (at 7.62 5.08 90) (size 1.6 1.6) (drill 0.8) (layers *.Cu *.Mask F.SilkS) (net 28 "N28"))
  (pad 27 thru_hole oval (at 7.62 2.54 90) (size 1.6 1.6) (drill 0.8) (layers *.Cu *.Mask F.SilkS) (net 2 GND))
  (pad 28 thru_hole oval (at 7.62 0 90) (size 1.6 1.6) (drill 0.8) (layers *.Cu *.Mask F.SilkS) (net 1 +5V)))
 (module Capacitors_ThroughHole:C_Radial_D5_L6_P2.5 (layer F.Cu) (at 69.215 71.12 270)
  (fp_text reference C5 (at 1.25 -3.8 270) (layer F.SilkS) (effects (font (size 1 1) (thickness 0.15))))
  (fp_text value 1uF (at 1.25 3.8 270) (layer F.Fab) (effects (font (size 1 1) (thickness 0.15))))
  (pad 1 thru_hole rect (at 0 0 270) (size 1.3 1.3) (drill 0.8) (layers *.Cu *.Mask F.SilkS) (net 7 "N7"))
  (pad 2 thru_hole circle (at 2.5 0 270) (size 1.3 1.3) (drill 0.8) (layers *.Cu *.Mask F.SilkS) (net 2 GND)))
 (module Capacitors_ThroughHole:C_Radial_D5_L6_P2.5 (layer F.Cu) (at 76.835 71.12 270)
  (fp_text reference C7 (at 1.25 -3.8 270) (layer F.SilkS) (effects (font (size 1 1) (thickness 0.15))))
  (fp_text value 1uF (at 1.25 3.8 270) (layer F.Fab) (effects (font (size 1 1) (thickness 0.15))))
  (pad 1 thru_hole rect (at 0 0 270) (size 1.3 1.3) (drill 0.8) (layers *.Cu *.Mask F.SilkS) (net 8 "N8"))
  (pad 2 thru_hole circle (at 2.5 0 270) (size 1.3 1.3) (drill 0.8) (layers *.Cu *.Mask F.SilkS) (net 2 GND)))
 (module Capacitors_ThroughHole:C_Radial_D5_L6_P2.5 (layer F.Cu) (at 115.57 46.99 270)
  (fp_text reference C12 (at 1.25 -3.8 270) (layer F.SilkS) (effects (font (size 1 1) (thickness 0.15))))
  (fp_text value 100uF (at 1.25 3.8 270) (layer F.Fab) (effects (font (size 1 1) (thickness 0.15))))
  (pad 1 thru_hole rect (at 0 0 270) (size 1.3 1.3) (drill 0.8) (layers *.Cu *.Mask F.SilkS) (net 1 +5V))
  (pad 2 thru_hole circle (at 2.5 0 270) (size 1.3 1.3) (drill 0.8) (layers *.Cu *.Mask F.SilkS) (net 2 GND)))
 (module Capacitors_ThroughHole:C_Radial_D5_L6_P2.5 (layer F.Cu) (at 142.24 46.99 270)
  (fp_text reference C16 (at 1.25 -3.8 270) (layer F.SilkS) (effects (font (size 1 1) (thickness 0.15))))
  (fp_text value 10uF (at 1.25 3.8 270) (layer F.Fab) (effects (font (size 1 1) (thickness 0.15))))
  (pad 1 thru_hole rect (at 0 0 270) (size 1.3 1.3) (drill 0.8) (layers *.Cu *.Mask F.SilkS) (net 11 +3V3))
  (pad 2 thru_hole circle (at 2.5 0 270) (size 1.3 1.3) (drill 0.8) (layers *.Cu *.Mask F.SilkS) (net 2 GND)))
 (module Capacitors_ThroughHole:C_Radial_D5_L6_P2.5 (layer F.Cu) (at 134.62 81.28 270)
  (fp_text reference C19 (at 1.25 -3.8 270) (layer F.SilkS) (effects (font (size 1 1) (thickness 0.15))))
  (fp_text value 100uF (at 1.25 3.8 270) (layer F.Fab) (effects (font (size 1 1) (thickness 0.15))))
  (pad 1 thru_hole rect (at 0 0 270) (size 1.3 1.3) (drill 0.8) (layers *.Cu *.Mask F.SilkS) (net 1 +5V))
  (pad 2 thru_hole circle (at 2.5 0 270) (size 1.3 1.3) (drill 0.8) (layers *.Cu *.Mask F.SilkS) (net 2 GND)))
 (gr_line (start 49.53 40.64) (end 49.53 90.17) (angle 90) (layer Edge.Cuts) (width 0.015))
 (gr_line (start 157.48 40.64) (end 49.53 40.64) (angle 90) (layer Edge.Cuts) (width 0.015))
 (gr_line (start 157.48 90.17) (end 157.48 40.64) (angle 90) (layer Edge.Cuts) (width 0.015))
 (gr_line (start 49.53 90.17) (end 157.48 90.17) (angle 90) (layer Edge.Cuts) (width 0.015))
 (segment (start 146.304 56.896) (end 146.05 57.15) (width 0.5) (layer B.Cu) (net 1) (status 30))
 (segment (start 87.55126 83.185) (end 87.63 83.185) (width 0.5) (layer B.Cu) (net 2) (status 30))
 (segment (start 120.015 73.56094) (end 120.11406 73.66) (width 0.5) (layer B.Cu) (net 31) (status 30))
 (segment (start 120.015 73.56094) (end 120.11406 73.66) (width 0.5) (layer B.Cu) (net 31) (status 30))
 (segment (start 125.095 73.56094) (end 124.99594 73.66) (width 0.5) (layer B.Cu) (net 32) (status 30)))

